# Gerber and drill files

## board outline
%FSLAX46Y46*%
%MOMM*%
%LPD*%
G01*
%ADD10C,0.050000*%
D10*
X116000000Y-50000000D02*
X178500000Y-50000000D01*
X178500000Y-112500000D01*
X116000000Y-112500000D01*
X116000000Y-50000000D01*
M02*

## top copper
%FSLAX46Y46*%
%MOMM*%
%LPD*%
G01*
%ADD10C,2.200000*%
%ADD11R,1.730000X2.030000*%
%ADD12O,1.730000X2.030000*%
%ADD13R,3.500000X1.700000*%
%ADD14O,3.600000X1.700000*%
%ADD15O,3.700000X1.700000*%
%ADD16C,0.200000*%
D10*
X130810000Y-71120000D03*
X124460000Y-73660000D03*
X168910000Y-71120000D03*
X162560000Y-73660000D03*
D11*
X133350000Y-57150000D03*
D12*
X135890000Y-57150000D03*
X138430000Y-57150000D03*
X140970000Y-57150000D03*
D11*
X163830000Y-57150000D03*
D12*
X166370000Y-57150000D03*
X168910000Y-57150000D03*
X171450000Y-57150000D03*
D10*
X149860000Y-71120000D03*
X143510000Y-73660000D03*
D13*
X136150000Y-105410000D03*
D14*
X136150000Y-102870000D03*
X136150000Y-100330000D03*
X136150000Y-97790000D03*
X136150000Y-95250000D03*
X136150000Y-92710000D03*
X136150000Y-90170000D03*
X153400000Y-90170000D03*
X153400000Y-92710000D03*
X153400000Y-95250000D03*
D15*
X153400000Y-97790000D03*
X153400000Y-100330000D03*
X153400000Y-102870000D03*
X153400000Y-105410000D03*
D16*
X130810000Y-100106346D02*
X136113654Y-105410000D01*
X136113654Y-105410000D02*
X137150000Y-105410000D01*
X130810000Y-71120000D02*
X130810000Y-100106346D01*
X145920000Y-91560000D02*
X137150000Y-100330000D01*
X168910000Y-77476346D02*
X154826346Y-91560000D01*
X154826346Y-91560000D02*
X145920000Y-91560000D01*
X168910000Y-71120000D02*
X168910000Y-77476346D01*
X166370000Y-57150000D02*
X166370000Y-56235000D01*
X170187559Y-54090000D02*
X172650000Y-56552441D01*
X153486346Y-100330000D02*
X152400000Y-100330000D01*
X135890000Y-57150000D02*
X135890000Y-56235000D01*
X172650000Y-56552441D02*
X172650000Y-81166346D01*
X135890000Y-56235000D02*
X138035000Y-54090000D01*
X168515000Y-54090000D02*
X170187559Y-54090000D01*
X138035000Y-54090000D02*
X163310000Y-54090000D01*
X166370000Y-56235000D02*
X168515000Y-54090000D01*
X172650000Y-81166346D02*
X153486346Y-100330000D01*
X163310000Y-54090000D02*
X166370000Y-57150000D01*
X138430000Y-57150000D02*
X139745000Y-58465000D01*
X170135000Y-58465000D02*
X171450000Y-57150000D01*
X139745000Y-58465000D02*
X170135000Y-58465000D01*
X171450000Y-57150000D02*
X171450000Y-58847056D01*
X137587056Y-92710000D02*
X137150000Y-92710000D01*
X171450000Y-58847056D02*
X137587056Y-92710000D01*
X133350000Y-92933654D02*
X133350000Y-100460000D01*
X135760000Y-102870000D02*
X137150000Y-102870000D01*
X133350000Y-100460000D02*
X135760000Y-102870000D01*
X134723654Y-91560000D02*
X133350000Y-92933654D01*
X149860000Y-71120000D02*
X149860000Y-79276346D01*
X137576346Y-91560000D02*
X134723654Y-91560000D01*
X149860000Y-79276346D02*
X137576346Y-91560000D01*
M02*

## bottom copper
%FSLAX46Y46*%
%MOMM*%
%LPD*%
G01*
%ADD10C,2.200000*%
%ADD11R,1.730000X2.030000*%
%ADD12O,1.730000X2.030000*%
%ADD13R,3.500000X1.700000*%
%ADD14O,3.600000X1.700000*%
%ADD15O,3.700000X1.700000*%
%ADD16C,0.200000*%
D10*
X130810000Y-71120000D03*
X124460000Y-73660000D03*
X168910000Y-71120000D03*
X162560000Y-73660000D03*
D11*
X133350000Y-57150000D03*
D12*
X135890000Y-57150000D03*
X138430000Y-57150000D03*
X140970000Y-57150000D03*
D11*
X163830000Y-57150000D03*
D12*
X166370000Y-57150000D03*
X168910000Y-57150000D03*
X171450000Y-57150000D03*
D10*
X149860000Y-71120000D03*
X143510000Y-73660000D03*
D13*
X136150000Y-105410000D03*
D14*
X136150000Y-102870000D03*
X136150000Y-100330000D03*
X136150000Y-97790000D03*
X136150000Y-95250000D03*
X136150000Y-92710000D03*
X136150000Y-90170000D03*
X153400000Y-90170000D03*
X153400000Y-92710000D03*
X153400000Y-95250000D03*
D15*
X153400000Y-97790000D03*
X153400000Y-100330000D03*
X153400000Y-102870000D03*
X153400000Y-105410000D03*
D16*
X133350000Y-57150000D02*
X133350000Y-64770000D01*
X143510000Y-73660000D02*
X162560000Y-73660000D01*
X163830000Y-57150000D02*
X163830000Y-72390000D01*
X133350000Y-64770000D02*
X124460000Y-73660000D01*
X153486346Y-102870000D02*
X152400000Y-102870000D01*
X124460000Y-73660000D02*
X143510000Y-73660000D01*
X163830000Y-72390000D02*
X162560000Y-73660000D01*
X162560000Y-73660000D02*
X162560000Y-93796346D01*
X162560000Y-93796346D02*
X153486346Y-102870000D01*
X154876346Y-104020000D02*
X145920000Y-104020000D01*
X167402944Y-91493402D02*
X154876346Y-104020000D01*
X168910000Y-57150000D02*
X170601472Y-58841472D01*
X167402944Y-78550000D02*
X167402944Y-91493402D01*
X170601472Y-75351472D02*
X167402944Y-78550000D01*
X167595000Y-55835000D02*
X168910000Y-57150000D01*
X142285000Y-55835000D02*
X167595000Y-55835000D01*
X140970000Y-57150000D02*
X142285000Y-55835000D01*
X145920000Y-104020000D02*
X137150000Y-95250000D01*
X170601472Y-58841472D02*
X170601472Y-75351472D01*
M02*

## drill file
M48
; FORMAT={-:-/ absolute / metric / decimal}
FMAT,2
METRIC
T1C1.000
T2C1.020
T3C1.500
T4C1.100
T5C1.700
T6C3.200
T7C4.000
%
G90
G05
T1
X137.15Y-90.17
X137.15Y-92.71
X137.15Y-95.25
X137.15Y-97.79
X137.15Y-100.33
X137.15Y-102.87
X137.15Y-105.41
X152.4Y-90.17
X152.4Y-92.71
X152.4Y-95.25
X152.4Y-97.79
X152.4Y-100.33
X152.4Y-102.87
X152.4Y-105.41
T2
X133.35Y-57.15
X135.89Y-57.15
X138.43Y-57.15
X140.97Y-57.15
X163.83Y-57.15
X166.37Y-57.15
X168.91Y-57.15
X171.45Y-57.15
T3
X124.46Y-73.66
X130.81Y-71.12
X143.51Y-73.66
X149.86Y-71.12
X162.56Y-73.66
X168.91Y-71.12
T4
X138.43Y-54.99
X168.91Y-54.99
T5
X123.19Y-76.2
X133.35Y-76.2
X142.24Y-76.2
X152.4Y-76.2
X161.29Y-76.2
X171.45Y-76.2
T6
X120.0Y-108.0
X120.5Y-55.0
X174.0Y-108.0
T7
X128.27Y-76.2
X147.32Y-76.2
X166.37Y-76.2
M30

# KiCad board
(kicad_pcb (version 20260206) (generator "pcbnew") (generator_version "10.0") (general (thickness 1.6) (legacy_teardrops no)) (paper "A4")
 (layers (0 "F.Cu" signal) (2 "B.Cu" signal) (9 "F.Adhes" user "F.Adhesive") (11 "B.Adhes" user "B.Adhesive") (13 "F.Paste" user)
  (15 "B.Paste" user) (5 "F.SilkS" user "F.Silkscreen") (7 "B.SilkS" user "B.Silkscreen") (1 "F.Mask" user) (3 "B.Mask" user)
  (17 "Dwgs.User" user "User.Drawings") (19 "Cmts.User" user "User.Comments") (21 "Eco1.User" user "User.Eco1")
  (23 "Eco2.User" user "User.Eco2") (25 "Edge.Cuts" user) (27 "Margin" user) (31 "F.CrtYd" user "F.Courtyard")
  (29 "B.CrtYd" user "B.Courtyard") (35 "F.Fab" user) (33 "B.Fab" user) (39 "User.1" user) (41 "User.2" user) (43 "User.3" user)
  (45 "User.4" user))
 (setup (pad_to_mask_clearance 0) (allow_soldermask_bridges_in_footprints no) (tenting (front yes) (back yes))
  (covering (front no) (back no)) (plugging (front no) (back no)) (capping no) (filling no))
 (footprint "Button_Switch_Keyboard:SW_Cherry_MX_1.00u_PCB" (layer "F.Cu") (at 130.81 71.12)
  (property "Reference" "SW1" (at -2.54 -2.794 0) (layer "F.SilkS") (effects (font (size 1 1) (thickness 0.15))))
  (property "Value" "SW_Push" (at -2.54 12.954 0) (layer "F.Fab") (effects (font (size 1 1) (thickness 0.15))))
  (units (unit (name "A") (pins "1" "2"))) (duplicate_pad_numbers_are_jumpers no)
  (pad "" np_thru_hole circle (at -7.62 5.08) (size 1.7 1.7) (drill 1.7) (layers "*.Cu" "*.Mask"))
  (pad "" np_thru_hole circle (at -2.54 5.08) (size 4 4) (drill 4) (layers "*.Cu" "*.Mask"))
  (pad "" np_thru_hole circle (at 2.54 5.08) (size 1.7 1.7) (drill 1.7) (layers "*.Cu" "*.Mask"))
  (pad "1" thru_hole circle (at 0 0) (size 2.2 2.2) (drill 1.5) (layers "*.Cu" "*.Mask") (remove_unused_layers no) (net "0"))
  (pad "2" thru_hole circle (at -6.35 2.54) (size 2.2 2.2) (drill 1.5) (layers "*.Cu" "*.Mask") (remove_unused_layers no) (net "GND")))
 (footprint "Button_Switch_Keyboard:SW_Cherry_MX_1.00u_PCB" (layer "F.Cu") (at 168.91 71.12)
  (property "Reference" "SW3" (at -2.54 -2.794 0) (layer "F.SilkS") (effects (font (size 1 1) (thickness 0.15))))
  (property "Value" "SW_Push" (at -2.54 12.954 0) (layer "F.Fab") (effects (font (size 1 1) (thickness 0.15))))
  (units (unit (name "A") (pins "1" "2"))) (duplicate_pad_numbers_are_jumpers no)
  (pad "" np_thru_hole circle (at -7.62 5.08) (size 1.7 1.7) (drill 1.7) (layers "*.Cu" "*.Mask"))
  (pad "" np_thru_hole circle (at -2.54 5.08) (size 4 4) (drill 4) (layers "*.Cu" "*.Mask"))
  (pad "" np_thru_hole circle (at 2.54 5.08) (size 1.7 1.7) (drill 1.7) (layers "*.Cu" "*.Mask"))
  (pad "1" thru_hole circle (at 0 0) (size 2.2 2.2) (drill 1.5) (layers "*.Cu" "*.Mask") (remove_unused_layers no) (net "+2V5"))
  (pad "2" thru_hole circle (at -6.35 2.54) (size 2.2 2.2) (drill 1.5) (layers "*.Cu" "*.Mask") (remove_unused_layers no) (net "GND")))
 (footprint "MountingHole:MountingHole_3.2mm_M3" (layer "F.Cu") (at 174 108)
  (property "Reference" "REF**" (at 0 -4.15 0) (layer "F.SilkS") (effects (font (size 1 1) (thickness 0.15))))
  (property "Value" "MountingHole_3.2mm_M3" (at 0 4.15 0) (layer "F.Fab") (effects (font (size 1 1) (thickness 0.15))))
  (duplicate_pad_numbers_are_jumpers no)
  (pad "" np_thru_hole circle (at 0 0) (size 3.2 3.2) (drill 3.2) (layers "*.Cu" "*.Mask")))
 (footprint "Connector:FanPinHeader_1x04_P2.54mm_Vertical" (layer "F.Cu") (at 133.35 57.15)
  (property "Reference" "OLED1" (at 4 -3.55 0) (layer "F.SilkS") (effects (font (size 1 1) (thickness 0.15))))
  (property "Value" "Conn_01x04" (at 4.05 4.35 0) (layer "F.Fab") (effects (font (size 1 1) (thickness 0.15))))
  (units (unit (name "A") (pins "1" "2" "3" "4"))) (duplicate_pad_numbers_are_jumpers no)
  (pad "" np_thru_hole circle (at 5.08 -2.16 90) (size 1.1 1.1) (drill 1.1) (layers "*.Cu" "*.Mask"))
  (pad "1" thru_hole rect (at 0 0 90) (size 2.03 1.73) (drill 1.02) (layers "*.Cu" "*.Mask") (remove_unused_layers no) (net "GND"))
  (pad "2" thru_hole oval (at 2.54 0 90) (size 2.03 1.73) (drill 1.02) (layers "*.Cu" "*.Mask") (remove_unused_layers no) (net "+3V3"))
  (pad "3" thru_hole oval (at 5.08 0 90) (size 2.03 1.73) (drill 1.02) (layers "*.Cu" "*.Mask") (remove_unused_layers no) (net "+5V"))
  (pad "4" thru_hole oval (at 7.62 0 90) (size 2.03 1.73) (drill 1.02) (layers "*.Cu" "*.Mask") (remove_unused_layers no) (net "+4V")))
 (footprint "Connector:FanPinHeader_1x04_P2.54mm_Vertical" (layer "F.Cu") (at 163.83 57.15)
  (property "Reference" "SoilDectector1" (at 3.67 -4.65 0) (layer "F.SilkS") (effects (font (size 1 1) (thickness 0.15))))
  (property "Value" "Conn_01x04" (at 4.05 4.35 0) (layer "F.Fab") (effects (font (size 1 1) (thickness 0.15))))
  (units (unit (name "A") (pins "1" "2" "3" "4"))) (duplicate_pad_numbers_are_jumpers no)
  (pad "" np_thru_hole circle (at 5.08 -2.16 90) (size 1.1 1.1) (drill 1.1) (layers "*.Cu" "*.Mask"))
  (pad "1" thru_hole rect (at 0 0 90) (size 2.03 1.73) (drill 1.02) (layers "*.Cu" "*.Mask") (remove_unused_layers no) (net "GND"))
  (pad "2" thru_hole oval (at 2.54 0 90) (size 2.03 1.73) (drill 1.02) (layers "*.Cu" "*.Mask") (remove_unused_layers no) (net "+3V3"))
  (pad "3" thru_hole oval (at 5.08 0 90) (size 2.03 1.73) (drill 1.02) (layers "*.Cu" "*.Mask") (remove_unused_layers no) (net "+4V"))
  (pad "4" thru_hole oval (at 7.62 0 90) (size 2.03 1.73) (drill 1.02) (layers "*.Cu" "*.Mask") (remove_unused_layers no) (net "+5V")))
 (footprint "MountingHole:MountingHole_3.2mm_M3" (layer "F.Cu") (at 120.5 55)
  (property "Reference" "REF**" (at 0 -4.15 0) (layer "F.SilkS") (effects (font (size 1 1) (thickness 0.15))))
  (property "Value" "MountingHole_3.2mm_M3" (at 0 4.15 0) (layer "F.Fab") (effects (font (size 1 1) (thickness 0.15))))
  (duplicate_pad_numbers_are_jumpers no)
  (pad "" np_thru_hole circle (at 0 0) (size 3.2 3.2) (drill 3.2) (layers "*.Cu" "*.Mask")))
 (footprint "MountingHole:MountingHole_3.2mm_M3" (layer "F.Cu") (at 120 108)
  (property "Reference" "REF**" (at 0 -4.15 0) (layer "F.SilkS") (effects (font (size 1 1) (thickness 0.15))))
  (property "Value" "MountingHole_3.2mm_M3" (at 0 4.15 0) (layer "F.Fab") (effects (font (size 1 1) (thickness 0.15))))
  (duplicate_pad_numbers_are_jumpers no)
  (pad "" np_thru_hole circle (at 0 0) (size 3.2 3.2) (drill 3.2) (layers "*.Cu" "*.Mask")))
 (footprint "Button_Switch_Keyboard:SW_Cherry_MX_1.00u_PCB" (layer "F.Cu") (at 149.86 71.12)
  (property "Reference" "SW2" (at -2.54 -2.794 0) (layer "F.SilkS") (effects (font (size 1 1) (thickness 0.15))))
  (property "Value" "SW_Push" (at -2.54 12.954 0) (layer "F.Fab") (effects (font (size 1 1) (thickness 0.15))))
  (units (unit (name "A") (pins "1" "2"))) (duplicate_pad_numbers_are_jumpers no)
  (pad "" np_thru_hole circle (at -7.62 5.08) (size 1.7 1.7) (drill 1.7) (layers "*.Cu" "*.Mask"))
  (pad "" np_thru_hole circle (at -2.54 5.08) (size 4 4) (drill 4) (layers "*.Cu" "*.Mask"))
  (pad "" np_thru_hole circle (at 2.54 5.08) (size 1.7 1.7) (drill 1.7) (layers "*.Cu" "*.Mask"))
  (pad "1" thru_hole circle (at 0 0) (size 2.2 2.2) (drill 1.5) (layers "*.Cu" "*.Mask") (remove_unused_layers no) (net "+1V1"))
  (pad "2" thru_hole circle (at -6.35 2.54) (size 2.2 2.2) (drill 1.5) (layers "*.Cu" "*.Mask") (remove_unused_layers no) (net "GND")))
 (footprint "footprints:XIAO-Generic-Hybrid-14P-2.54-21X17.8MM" (layer "B.Cu") (at 144.775 97.79)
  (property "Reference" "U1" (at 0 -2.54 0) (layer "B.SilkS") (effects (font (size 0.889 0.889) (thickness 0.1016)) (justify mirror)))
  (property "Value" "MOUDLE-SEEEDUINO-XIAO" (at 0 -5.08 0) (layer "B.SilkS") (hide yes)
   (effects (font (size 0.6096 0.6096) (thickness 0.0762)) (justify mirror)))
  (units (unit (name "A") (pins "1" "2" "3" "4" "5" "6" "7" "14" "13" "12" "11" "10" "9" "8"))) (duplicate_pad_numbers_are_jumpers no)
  (pad "1" thru_hole rect (at -7.625 7.62) (size 3.5 1.7) (drill 1 (offset -1 0)) (layers "*.Cu" "*.Mask") (remove_unused_layers no)
   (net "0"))
  (pad "2" thru_hole oval (at -7.625 5.08) (size 3.6 1.7) (drill 1 (offset -1 0)) (layers "*.Cu" "*.Mask") (remove_unused_layers no)
   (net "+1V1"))
  (pad "3" thru_hole oval (at -7.625 2.54) (size 3.6 1.7) (drill 1 (offset -1 0)) (layers "*.Cu" "*.Mask") (remove_unused_layers no)
   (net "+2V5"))
  (pad "4" thru_hole oval (at -7.625 0) (size 3.6 1.7) (drill 1 (offset -1 0)) (layers "*.Cu" "*.Mask") (remove_unused_layers no)
   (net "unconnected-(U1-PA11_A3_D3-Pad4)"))
  (pad "5" thru_hole oval (at -7.625 -2.54) (size 3.6 1.7) (drill 1 (offset -1 0)) (layers "*.Cu" "*.Mask") (remove_unused_layers no)
   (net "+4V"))
  (pad "6" thru_hole oval (at -7.625 -5.08 180) (size 3.6 1.7) (drill 1 (offset 1 0)) (layers "*.Cu" "*.Mask") (remove_unused_layers no)
   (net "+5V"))
  (pad "7" thru_hole oval (at -7.625 -7.62) (size 3.6 1.7) (drill 1 (offset -1 0)) (layers "*.Cu" "*.Mask") (remove_unused_layers no)
   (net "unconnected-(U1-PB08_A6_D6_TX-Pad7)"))
  (pad "8" thru_hole oval (at 7.625 -7.62) (size 3.6 1.7) (drill 1 (offset 1 0)) (layers "*.Cu" "*.Mask") (remove_unused_layers no)
   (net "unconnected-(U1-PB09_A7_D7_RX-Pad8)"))
  (pad "9" thru_hole oval (at 7.625 -5.08) (size 3.6 1.7) (drill 1 (offset 1 0)) (layers "*.Cu" "*.Mask") (remove_unused_layers no)
   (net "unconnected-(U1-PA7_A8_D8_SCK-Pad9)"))
  (pad "10" thru_hole oval (at 7.625 -2.54) (size 3.6 1.7) (drill 1 (offset 1 0)) (layers "*.Cu" "*.Mask") (remove_unused_layers no)
   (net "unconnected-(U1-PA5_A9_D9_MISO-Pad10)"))
  (pad "11" thru_hole oval (at 7.625 0) (size 3.7 1.7) (drill 1 (offset 1 0)) (layers "*.Cu" "*.Mask") (remove_unused_layers no)
   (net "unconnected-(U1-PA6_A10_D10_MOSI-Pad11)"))
  (pad "12" thru_hole oval (at 7.625 2.54) (size 3.7 1.7) (drill 1 (offset 1 0)) (layers "*.Cu" "*.Mask") (remove_unused_layers no)
   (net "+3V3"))
  (pad "13" thru_hole oval (at 7.625 5.08) (size 3.7 1.7) (drill 1 (offset 1 0)) (layers "*.Cu" "*.Mask") (remove_unused_layers no)
   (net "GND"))
  (pad "14" thru_hole oval (at 7.625 7.62) (size 3.7 1.7) (drill 1 (offset 1 0)) (layers "*.Cu" "*.Mask") (remove_unused_layers no)
   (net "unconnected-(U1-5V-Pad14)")))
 (gr_rect (start 116 50) (end 178.5 112.5) (stroke (width 0.05) (type default)) (fill no) (layer "Edge.Cuts"))
 (segment (start 130.81 100.106346) (end 136.113654 105.41) (width 0.2) (layer "F.Cu") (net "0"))
 (segment (start 136.113654 105.41) (end 137.15 105.41) (width 0.2) (layer "F.Cu") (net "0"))
 (segment (start 130.81 71.12) (end 130.81 100.106346) (width 0.2) (layer "F.Cu") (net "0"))
 (segment (start 133.35 57.15) (end 133.35 64.77) (width 0.2) (layer "B.Cu") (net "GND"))
 (segment (start 143.51 73.66) (end 162.56 73.66) (width 0.2) (layer "B.Cu") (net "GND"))
 (segment (start 163.83 57.15) (end 163.83 72.39) (width 0.2) (layer "B.Cu") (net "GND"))
 (segment (start 133.35 64.77) (end 124.46 73.66) (width 0.2) (layer "B.Cu") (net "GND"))
 (segment (start 153.486346 102.87) (end 152.4 102.87) (width 0.2) (layer "B.Cu") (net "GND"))
 (segment (start 124.46 73.66) (end 143.51 73.66) (width 0.2) (layer "B.Cu") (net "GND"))
 (segment (start 163.83 72.39) (end 162.56 73.66) (width 0.2) (layer "B.Cu") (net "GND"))
 (segment (start 162.56 73.66) (end 162.56 93.796346) (width 0.2) (layer "B.Cu") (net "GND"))
 (segment (start 162.56 93.796346) (end 153.486346 102.87) (width 0.2) (layer "B.Cu") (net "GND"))
 (segment (start 145.92 91.56) (end 137.15 100.33) (width 0.2) (layer "F.Cu") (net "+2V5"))
 (segment (start 168.91 77.476346) (end 154.826346 91.56) (width 0.2) (layer "F.Cu") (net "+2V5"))
 (segment (start 154.826346 91.56) (end 145.92 91.56) (width 0.2) (layer "F.Cu") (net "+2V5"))
 (segment (start 168.91 71.12) (end 168.91 77.476346) (width 0.2) (layer "F.Cu") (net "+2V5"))
 (segment (start 166.37 57.15) (end 166.37 56.235) (width 0.2) (layer "F.Cu") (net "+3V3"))
 (segment (start 170.187559 54.09) (end 172.65 56.552441) (width 0.2) (layer "F.Cu") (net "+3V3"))
 (segment (start 153.486346 100.33) (end 152.4 100.33) (width 0.2) (layer "F.Cu") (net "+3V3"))
 (segment (start 135.89 57.15) (end 135.89 56.235) (width 0.2) (layer "F.Cu") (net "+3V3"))
 (segment (start 172.65 56.552441) (end 172.65 81.166346) (width 0.2) (layer "F.Cu") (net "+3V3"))
 (segment (start 135.89 56.235) (end 138.035 54.09) (width 0.2) (layer "F.Cu") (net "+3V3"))
 (segment (start 168.515 54.09) (end 170.187559 54.09) (width 0.2) (layer "F.Cu") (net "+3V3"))
 (segment (start 138.035 54.09) (end 163.31 54.09) (width 0.2) (layer "F.Cu") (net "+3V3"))
 (segment (start 166.37 56.235) (end 168.515 54.09) (width 0.2) (layer "F.Cu") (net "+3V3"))
 (segment (start 172.65 81.166346) (end 153.486346 100.33) (width 0.2) (layer "F.Cu") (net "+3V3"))
 (segment (start 163.31 54.09) (end 166.37 57.15) (width 0.2) (layer "F.Cu") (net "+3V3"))
 (segment (start 138.43 57.15) (end 139.745 58.465) (width 0.2) (layer "F.Cu") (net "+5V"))
 (segment (start 170.135 58.465) (end 171.45 57.15) (width 0.2) (layer "F.Cu") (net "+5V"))
 (segment (start 139.745 58.465) (end 170.135 58.465) (width 0.2) (layer "F.Cu") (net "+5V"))
 (segment (start 171.45 57.15) (end 171.45 58.847056) (width 0.2) (layer "F.Cu") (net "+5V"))
 (segment (start 137.587056 92.71) (end 137.15 92.71) (width 0.2) (layer "F.Cu") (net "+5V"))
 (segment (start 171.45 58.847056) (end 137.587056 92.71) (width 0.2) (layer "F.Cu") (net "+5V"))
 (segment (start 154.876346 104.02) (end 145.92 104.02) (width 0.2) (layer "B.Cu") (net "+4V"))
 (segment (start 167.402944 91.493402) (end 154.876346 104.02) (width 0.2) (layer "B.Cu") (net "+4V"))
 (segment (start 168.91 57.15) (end 170.601472 58.841472) (width 0.2) (layer "B.Cu") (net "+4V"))
 (segment (start 167.402944 78.55) (end 167.402944 91.493402) (width 0.2) (layer "B.Cu") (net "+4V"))
 (segment (start 170.601472 75.351472) (end 167.402944 78.55) (width 0.2) (layer "B.Cu") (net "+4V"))
 (segment (start 167.595 55.835) (end 168.91 57.15) (width 0.2) (layer "B.Cu") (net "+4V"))
 (segment (start 142.285 55.835) (end 167.595 55.835) (width 0.2) (layer "B.Cu") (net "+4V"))
 (segment (start 140.97 57.15) (end 142.285 55.835) (width 0.2) (layer "B.Cu") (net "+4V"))
 (segment (start 145.92 104.02) (end 137.15 95.25) (width 0.2) (layer "B.Cu") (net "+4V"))
 (segment (start 170.601472 58.841472) (end 170.601472 75.351472) (width 0.2) (layer "B.Cu") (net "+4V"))
 (segment (start 133.35 92.933654) (end 133.35 100.46) (width 0.2) (layer "F.Cu") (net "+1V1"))
 (segment (start 135.76 102.87) (end 137.15 102.87) (width 0.2) (layer "F.Cu") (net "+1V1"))
 (segment (start 133.35 100.46) (end 135.76 102.87) (width 0.2) (layer "F.Cu") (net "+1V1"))
 (segment (start 134.723654 91.56) (end 133.35 92.933654) (width 0.2) (layer "F.Cu") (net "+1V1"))
 (segment (start 149.86 71.12) (end 149.86 79.276346) (width 0.2) (layer "F.Cu") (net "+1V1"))
 (segment (start 137.576346 91.56) (end 134.723654 91.56) (width 0.2) (layer "F.Cu") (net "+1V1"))
 (segment (start 149.86 79.276346) (end 137.576346 91.56) (width 0.2) (layer "F.Cu") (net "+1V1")))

